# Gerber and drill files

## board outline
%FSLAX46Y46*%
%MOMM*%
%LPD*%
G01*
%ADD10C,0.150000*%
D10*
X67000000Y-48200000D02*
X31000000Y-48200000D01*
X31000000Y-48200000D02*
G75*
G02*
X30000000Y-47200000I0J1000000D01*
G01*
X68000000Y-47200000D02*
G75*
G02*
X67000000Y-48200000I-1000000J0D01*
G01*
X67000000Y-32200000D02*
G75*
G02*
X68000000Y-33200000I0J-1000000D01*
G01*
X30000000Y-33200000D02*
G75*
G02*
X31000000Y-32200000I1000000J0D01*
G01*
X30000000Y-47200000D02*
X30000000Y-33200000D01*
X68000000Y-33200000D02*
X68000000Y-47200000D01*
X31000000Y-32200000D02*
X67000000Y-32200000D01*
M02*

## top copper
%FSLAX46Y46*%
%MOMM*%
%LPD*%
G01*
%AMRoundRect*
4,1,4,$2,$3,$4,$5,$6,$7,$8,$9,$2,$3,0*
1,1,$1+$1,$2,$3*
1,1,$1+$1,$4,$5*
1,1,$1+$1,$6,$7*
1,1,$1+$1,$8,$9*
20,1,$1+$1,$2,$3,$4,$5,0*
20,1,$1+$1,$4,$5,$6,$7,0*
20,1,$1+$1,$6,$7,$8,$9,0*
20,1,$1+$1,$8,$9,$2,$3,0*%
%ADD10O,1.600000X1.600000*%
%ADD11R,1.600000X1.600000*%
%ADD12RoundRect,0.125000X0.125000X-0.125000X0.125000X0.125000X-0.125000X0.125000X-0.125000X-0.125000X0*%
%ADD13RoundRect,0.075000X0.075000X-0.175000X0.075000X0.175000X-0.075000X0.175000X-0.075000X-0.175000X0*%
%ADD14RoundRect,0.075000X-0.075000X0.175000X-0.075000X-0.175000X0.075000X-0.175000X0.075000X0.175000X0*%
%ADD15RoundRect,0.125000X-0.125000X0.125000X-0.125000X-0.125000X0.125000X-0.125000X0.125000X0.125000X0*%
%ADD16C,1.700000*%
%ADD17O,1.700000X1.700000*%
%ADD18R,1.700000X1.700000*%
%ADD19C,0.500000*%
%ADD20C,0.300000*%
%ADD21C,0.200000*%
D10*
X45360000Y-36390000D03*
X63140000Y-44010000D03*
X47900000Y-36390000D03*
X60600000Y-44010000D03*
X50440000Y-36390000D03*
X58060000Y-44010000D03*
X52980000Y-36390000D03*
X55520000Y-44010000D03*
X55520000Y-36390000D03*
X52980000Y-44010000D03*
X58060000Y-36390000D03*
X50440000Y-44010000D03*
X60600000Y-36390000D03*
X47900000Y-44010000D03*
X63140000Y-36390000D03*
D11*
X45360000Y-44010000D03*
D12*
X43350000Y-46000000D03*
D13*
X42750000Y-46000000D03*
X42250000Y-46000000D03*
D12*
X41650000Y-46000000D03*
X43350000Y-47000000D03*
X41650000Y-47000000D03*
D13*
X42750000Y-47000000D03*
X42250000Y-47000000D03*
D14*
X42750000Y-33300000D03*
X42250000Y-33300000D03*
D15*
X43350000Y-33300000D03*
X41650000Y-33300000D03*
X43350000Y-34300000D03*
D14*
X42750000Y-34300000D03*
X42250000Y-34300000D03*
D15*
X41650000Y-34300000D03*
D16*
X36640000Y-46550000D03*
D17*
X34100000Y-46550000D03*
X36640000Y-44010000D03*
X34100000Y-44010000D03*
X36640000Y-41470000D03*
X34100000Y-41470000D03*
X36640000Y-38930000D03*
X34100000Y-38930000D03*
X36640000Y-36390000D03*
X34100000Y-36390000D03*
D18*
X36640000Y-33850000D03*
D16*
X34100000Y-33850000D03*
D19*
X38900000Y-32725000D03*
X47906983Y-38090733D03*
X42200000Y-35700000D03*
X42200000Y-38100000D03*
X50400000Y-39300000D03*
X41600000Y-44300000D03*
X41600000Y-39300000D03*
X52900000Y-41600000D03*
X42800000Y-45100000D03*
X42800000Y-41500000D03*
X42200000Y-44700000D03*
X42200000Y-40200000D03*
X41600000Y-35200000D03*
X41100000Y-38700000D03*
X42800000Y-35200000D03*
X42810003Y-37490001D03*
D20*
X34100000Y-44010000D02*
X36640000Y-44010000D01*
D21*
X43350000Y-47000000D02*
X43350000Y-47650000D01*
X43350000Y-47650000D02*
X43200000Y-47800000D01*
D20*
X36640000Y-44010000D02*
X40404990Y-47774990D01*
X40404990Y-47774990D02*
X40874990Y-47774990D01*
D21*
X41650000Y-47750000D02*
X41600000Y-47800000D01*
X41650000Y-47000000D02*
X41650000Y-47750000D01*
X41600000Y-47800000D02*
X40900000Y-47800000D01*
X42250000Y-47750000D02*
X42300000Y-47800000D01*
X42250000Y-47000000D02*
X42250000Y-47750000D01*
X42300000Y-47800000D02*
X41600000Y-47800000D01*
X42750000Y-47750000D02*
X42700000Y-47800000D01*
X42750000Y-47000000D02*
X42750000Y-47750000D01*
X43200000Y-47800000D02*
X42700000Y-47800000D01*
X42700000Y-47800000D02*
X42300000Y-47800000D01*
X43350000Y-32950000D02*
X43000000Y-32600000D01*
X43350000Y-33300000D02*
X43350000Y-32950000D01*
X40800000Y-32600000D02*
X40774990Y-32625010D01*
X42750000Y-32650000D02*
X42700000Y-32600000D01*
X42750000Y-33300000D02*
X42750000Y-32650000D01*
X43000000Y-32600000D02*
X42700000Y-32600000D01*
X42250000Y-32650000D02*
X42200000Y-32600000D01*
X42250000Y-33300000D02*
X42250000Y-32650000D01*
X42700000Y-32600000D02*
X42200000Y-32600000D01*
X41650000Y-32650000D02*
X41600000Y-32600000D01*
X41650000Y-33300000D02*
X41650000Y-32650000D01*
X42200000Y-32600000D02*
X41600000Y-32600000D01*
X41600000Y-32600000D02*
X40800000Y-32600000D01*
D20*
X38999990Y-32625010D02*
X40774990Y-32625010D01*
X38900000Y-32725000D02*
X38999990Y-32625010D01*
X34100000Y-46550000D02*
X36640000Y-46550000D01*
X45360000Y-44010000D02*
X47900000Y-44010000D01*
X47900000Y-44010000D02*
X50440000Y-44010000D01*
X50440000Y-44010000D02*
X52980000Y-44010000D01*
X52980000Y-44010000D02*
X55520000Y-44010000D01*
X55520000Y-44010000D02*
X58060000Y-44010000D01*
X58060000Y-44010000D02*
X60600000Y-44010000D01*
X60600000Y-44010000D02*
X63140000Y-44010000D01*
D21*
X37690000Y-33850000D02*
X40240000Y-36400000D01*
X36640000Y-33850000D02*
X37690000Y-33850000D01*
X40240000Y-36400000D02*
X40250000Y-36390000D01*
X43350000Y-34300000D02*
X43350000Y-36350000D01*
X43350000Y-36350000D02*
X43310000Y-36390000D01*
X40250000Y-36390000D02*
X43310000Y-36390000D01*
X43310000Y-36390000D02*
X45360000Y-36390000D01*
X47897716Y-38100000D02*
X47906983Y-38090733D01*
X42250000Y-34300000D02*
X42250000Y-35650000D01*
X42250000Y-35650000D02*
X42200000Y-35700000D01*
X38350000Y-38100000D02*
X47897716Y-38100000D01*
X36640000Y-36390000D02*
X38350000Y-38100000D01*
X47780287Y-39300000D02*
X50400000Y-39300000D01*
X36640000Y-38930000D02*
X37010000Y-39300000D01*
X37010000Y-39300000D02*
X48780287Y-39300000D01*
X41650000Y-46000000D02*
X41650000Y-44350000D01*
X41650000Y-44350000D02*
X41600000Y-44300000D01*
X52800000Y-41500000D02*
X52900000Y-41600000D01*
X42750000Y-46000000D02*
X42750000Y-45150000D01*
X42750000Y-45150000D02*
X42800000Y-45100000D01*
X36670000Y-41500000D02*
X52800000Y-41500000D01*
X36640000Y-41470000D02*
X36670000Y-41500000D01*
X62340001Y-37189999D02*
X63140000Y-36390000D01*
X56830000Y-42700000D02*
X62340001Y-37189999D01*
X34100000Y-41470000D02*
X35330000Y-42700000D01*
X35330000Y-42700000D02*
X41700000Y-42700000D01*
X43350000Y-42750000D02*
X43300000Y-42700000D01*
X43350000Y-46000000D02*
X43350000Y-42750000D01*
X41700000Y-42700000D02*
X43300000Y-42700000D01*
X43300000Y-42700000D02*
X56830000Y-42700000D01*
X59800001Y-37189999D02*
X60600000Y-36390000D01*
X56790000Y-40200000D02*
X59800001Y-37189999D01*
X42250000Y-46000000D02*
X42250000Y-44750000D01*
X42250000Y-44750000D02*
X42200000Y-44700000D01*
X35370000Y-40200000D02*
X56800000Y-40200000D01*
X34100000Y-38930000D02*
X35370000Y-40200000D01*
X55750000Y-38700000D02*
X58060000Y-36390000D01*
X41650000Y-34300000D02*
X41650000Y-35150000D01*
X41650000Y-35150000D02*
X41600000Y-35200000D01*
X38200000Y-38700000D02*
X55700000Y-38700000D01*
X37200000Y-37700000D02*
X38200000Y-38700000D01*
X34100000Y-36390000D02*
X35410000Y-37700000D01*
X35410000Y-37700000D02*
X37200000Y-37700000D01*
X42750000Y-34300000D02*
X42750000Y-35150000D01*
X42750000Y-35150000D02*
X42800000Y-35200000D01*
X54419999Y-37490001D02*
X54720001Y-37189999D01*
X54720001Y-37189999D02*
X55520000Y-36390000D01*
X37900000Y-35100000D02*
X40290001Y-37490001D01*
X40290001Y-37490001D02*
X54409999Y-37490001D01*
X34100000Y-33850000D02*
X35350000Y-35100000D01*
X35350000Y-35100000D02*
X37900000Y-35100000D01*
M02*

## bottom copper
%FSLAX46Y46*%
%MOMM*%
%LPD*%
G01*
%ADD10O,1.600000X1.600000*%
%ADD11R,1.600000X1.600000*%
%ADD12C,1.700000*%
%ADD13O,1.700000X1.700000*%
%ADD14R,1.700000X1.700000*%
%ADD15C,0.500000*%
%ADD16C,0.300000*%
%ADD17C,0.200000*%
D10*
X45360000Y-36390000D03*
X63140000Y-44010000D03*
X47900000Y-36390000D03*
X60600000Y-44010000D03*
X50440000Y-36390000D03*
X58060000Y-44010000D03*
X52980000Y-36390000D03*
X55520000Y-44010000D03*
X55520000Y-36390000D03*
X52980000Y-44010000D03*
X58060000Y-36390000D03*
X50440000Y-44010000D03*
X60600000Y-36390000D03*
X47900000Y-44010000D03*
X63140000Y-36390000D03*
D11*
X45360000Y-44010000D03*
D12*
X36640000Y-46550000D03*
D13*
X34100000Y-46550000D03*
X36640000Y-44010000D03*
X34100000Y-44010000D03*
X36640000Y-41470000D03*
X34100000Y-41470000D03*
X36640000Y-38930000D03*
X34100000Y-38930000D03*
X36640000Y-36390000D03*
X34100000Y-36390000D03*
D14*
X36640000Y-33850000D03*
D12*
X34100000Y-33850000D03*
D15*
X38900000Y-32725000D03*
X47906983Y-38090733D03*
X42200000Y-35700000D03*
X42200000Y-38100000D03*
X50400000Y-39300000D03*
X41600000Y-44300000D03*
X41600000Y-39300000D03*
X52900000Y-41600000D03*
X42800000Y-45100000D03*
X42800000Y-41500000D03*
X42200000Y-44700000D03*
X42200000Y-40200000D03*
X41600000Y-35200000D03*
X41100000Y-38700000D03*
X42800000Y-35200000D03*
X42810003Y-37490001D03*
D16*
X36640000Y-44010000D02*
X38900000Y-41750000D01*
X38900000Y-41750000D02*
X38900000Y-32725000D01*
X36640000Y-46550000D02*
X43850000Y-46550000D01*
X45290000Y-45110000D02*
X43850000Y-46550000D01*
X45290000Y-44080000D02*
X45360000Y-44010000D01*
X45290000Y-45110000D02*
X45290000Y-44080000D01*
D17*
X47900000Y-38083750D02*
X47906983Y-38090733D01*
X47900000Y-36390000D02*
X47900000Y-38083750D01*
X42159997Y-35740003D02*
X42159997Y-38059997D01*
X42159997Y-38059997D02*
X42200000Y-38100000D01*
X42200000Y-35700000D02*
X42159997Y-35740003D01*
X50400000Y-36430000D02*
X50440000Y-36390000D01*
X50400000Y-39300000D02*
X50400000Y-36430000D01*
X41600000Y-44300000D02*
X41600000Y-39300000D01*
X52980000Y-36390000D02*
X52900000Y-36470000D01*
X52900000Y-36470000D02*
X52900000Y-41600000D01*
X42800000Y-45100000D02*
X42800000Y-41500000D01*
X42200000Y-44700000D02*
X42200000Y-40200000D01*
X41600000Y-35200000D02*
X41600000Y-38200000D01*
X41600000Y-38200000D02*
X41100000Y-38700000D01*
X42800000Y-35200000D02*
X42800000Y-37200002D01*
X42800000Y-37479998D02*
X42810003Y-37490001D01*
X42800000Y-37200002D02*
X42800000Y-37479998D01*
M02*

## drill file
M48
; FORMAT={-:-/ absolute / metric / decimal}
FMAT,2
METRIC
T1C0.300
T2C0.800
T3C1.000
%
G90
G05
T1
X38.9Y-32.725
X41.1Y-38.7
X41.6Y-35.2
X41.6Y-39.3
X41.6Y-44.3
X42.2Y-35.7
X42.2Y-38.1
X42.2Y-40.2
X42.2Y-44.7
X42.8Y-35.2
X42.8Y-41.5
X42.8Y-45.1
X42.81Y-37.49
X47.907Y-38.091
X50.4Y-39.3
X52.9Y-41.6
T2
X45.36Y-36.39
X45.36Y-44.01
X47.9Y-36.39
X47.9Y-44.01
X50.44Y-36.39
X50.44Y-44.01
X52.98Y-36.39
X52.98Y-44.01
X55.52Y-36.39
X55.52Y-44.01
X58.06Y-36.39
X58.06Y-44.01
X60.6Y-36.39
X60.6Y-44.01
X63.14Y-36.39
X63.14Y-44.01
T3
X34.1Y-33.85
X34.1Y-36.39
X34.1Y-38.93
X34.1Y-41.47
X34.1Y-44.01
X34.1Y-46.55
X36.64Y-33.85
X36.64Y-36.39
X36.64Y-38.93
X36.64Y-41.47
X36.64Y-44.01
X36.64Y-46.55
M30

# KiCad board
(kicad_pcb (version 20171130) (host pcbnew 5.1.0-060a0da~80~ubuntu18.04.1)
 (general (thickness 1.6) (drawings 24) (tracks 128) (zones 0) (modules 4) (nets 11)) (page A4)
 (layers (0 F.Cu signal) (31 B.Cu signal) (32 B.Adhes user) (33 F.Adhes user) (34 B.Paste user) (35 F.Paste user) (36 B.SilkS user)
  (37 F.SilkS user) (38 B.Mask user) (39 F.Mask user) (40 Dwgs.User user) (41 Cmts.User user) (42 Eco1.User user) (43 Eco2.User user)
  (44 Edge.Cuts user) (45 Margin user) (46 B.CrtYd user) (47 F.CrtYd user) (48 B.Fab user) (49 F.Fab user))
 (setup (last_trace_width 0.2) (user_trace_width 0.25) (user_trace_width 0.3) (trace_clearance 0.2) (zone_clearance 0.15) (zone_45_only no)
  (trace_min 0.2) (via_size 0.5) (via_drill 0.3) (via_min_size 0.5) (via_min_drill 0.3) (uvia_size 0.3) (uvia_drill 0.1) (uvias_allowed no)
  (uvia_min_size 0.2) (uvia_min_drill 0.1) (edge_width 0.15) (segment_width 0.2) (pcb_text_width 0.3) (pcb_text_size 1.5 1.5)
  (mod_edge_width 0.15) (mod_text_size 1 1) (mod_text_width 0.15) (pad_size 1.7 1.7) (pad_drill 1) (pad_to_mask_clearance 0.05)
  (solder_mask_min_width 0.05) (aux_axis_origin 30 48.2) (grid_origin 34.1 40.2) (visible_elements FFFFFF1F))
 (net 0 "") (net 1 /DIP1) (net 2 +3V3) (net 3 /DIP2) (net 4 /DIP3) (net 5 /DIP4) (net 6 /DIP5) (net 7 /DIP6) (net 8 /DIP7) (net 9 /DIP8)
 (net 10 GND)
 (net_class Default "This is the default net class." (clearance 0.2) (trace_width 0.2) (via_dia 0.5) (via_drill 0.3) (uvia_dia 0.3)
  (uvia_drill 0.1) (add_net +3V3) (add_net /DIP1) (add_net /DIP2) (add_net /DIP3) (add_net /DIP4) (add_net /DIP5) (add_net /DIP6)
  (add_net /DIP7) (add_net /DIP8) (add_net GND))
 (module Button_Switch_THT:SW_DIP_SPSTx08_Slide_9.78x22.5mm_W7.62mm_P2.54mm (layer F.Cu) (at 45.36 44.01 90)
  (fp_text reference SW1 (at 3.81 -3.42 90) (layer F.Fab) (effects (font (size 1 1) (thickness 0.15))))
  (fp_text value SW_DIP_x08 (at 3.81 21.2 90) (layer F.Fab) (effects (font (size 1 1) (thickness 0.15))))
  (pad 16 thru_hole oval (at 7.62 0 90) (size 1.6 1.6) (drill 0.8) (layers *.Cu *.Mask) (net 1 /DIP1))
  (pad 8 thru_hole oval (at 0 17.78 90) (size 1.6 1.6) (drill 0.8) (layers *.Cu *.Mask) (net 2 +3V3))
  (pad 15 thru_hole oval (at 7.62 2.54 90) (size 1.6 1.6) (drill 0.8) (layers *.Cu *.Mask) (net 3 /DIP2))
  (pad 7 thru_hole oval (at 0 15.24 90) (size 1.6 1.6) (drill 0.8) (layers *.Cu *.Mask) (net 2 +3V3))
  (pad 14 thru_hole oval (at 7.62 5.08 90) (size 1.6 1.6) (drill 0.8) (layers *.Cu *.Mask) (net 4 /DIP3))
  (pad 6 thru_hole oval (at 0 12.7 90) (size 1.6 1.6) (drill 0.8) (layers *.Cu *.Mask) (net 2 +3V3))
  (pad 13 thru_hole oval (at 7.62 7.62 90) (size 1.6 1.6) (drill 0.8) (layers *.Cu *.Mask) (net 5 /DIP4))
  (pad 5 thru_hole oval (at 0 10.16 90) (size 1.6 1.6) (drill 0.8) (layers *.Cu *.Mask) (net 2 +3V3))
  (pad 12 thru_hole oval (at 7.62 10.16 90) (size 1.6 1.6) (drill 0.8) (layers *.Cu *.Mask) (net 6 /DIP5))
  (pad 4 thru_hole oval (at 0 7.62 90) (size 1.6 1.6) (drill 0.8) (layers *.Cu *.Mask) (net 2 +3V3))
  (pad 11 thru_hole oval (at 7.62 12.7 90) (size 1.6 1.6) (drill 0.8) (layers *.Cu *.Mask) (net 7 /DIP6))
  (pad 3 thru_hole oval (at 0 5.08 90) (size 1.6 1.6) (drill 0.8) (layers *.Cu *.Mask) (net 2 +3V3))
  (pad 10 thru_hole oval (at 7.62 15.24 90) (size 1.6 1.6) (drill 0.8) (layers *.Cu *.Mask) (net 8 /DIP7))
  (pad 2 thru_hole oval (at 0 2.54 90) (size 1.6 1.6) (drill 0.8) (layers *.Cu *.Mask) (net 2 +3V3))
  (pad 9 thru_hole oval (at 7.62 17.78 90) (size 1.6 1.6) (drill 0.8) (layers *.Cu *.Mask) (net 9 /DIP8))
  (pad 1 thru_hole rect (at 0 0 90) (size 1.6 1.6) (drill 0.8) (layers *.Cu *.Mask) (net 2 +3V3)))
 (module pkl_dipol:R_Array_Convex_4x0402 (layer F.Cu) (at 42.5 46.5 90) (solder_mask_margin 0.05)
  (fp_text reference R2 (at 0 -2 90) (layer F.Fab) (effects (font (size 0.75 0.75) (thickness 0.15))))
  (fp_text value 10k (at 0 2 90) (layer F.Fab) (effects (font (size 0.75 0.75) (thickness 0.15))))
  (pad 8 smd roundrect (at 0.5 0.85 90) (size 0.5 0.5) (layers F.Cu F.Paste F.Mask) (roundrect_rratio 0.25) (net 9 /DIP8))
  (pad 6 smd roundrect (at 0.5 0.25 90) (size 0.5 0.3) (layers F.Cu F.Paste F.Mask) (roundrect_rratio 0.25) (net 5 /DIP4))
  (pad 4 smd roundrect (at 0.5 -0.25 90) (size 0.5 0.3) (layers F.Cu F.Paste F.Mask) (roundrect_rratio 0.25) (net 8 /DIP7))
  (pad 2 smd roundrect (at 0.5 -0.85 90) (size 0.5 0.5) (layers F.Cu F.Paste F.Mask) (roundrect_rratio 0.25) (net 4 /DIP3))
  (pad 7 smd roundrect (at -0.5 0.85 90) (size 0.5 0.5) (layers F.Cu F.Paste F.Mask) (roundrect_rratio 0.25) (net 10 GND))
  (pad 1 smd roundrect (at -0.5 -0.85 90) (size 0.5 0.5) (layers F.Cu F.Paste F.Mask) (roundrect_rratio 0.25) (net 10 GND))
  (pad 5 smd roundrect (at -0.5 0.25 90) (size 0.5 0.3) (layers F.Cu F.Paste F.Mask) (roundrect_rratio 0.25) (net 10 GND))
  (pad 3 smd roundrect (at -0.5 -0.25 90) (size 0.5 0.3) (layers F.Cu F.Paste F.Mask) (roundrect_rratio 0.25) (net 10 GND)))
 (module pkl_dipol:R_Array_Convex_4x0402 (layer F.Cu) (at 42.5 33.8 270) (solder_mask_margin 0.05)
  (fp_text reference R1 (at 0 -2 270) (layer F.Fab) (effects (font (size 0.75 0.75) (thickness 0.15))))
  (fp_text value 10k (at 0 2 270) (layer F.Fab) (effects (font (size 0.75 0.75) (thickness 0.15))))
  (pad 3 smd roundrect (at -0.5 -0.25 270) (size 0.5 0.3) (layers F.Cu F.Paste F.Mask) (roundrect_rratio 0.25) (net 10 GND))
  (pad 5 smd roundrect (at -0.5 0.25 270) (size 0.5 0.3) (layers F.Cu F.Paste F.Mask) (roundrect_rratio 0.25) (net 10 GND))
  (pad 1 smd roundrect (at -0.5 -0.85 270) (size 0.5 0.5) (layers F.Cu F.Paste F.Mask) (roundrect_rratio 0.25) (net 10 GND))
  (pad 7 smd roundrect (at -0.5 0.85 270) (size 0.5 0.5) (layers F.Cu F.Paste F.Mask) (roundrect_rratio 0.25) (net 10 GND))
  (pad 2 smd roundrect (at 0.5 -0.85 270) (size 0.5 0.5) (layers F.Cu F.Paste F.Mask) (roundrect_rratio 0.25) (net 1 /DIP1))
  (pad 4 smd roundrect (at 0.5 -0.25 270) (size 0.5 0.3) (layers F.Cu F.Paste F.Mask) (roundrect_rratio 0.25) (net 6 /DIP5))
  (pad 6 smd roundrect (at 0.5 0.25 270) (size 0.5 0.3) (layers F.Cu F.Paste F.Mask) (roundrect_rratio 0.25) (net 3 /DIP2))
  (pad 8 smd roundrect (at 0.5 0.85 270) (size 0.5 0.5) (layers F.Cu F.Paste F.Mask) (roundrect_rratio 0.25) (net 7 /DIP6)))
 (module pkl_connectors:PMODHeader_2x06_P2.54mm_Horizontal (layer F.Cu) (at 36.64 46.55 180)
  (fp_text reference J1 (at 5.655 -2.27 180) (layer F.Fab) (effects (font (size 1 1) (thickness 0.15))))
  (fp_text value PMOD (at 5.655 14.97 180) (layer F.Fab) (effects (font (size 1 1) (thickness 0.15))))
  (pad 6 thru_hole circle (at 0 0 180) (size 1.7 1.7) (drill 1) (layers *.Cu *.Mask) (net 2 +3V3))
  (pad 12 thru_hole oval (at 2.54 0 180) (size 1.7 1.7) (drill 1) (layers *.Cu *.Mask) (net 2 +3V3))
  (pad 5 thru_hole oval (at 0 2.54 180) (size 1.7 1.7) (drill 1) (layers *.Cu *.Mask) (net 10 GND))
  (pad 11 thru_hole oval (at 2.54 2.54 180) (size 1.7 1.7) (drill 1) (layers *.Cu *.Mask) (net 10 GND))
  (pad 4 thru_hole oval (at 0 5.08 180) (size 1.7 1.7) (drill 1) (layers *.Cu *.Mask) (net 5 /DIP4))
  (pad 10 thru_hole oval (at 2.54 5.08 180) (size 1.7 1.7) (drill 1) (layers *.Cu *.Mask) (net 9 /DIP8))
  (pad 3 thru_hole oval (at 0 7.62 180) (size 1.7 1.7) (drill 1) (layers *.Cu *.Mask) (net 4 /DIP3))
  (pad 9 thru_hole oval (at 2.54 7.62 180) (size 1.7 1.7) (drill 1) (layers *.Cu *.Mask) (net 8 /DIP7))
  (pad 2 thru_hole oval (at 0 10.16 180) (size 1.7 1.7) (drill 1) (layers *.Cu *.Mask) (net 3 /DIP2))
  (pad 8 thru_hole oval (at 2.54 10.16 180) (size 1.7 1.7) (drill 1) (layers *.Cu *.Mask) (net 7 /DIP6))
  (pad 1 thru_hole rect (at 0 12.7 180) (size 1.7 1.7) (drill 1) (layers *.Cu *.Mask) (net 1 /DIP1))
  (pad 7 thru_hole circle (at 2.54 12.7 180) (size 1.7 1.7) (drill 1) (layers *.Cu *.Mask) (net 6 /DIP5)))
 (gr_line (start 67 48.2) (end 31 48.2) (layer Edge.Cuts) (width 0.15))
 (gr_arc (start 31 47.2) (end 30 47.2) (angle -90) (layer Edge.Cuts) (width 0.15))
 (gr_arc (start 67 47.2) (end 67 48.2) (angle -90) (layer Edge.Cuts) (width 0.15))
 (gr_arc (start 67 33.2) (end 68 33.2) (angle -90) (layer Edge.Cuts) (width 0.15))
 (gr_arc (start 31 33.2) (end 31 32.2) (angle -90) (layer Edge.Cuts) (width 0.15))
 (gr_line (start 30 47.2) (end 30 33.2) (layer Edge.Cuts) (width 0.15))
 (gr_line (start 68 33.2) (end 68 47.2) (layer Edge.Cuts) (width 0.15))
 (gr_line (start 31 32.2) (end 67 32.2) (layer Edge.Cuts) (width 0.15))
 (segment (start 34.1 44.01) (end 36.64 44.01) (width 0.3) (layer F.Cu) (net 10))
 (segment (start 43.35 47) (end 43.35 47.65) (width 0.2) (layer F.Cu) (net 10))
 (segment (start 43.35 47.65) (end 43.2 47.8) (width 0.2) (layer F.Cu) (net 10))
 (segment (start 36.64 44.01) (end 40.40499 47.77499) (width 0.3) (layer F.Cu) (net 10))
 (segment (start 40.40499 47.77499) (end 40.87499 47.77499) (width 0.3) (layer F.Cu) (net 10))
 (segment (start 41.65 47.75) (end 41.6 47.8) (width 0.2) (layer F.Cu) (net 10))
 (segment (start 41.65 47) (end 41.65 47.75) (width 0.2) (layer F.Cu) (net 10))
 (segment (start 41.6 47.8) (end 40.9 47.8) (width 0.2) (layer F.Cu) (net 10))
 (segment (start 42.25 47.75) (end 42.3 47.8) (width 0.2) (layer F.Cu) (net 10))
 (segment (start 42.25 47) (end 42.25 47.75) (width 0.2) (layer F.Cu) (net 10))
 (segment (start 42.3 47.8) (end 41.6 47.8) (width 0.2) (layer F.Cu) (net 10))
 (segment (start 42.75 47.75) (end 42.7 47.8) (width 0.2) (layer F.Cu) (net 10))
 (segment (start 42.75 47) (end 42.75 47.75) (width 0.2) (layer F.Cu) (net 10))
 (segment (start 43.2 47.8) (end 42.7 47.8) (width 0.2) (layer F.Cu) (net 10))
 (segment (start 42.7 47.8) (end 42.3 47.8) (width 0.2) (layer F.Cu) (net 10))
 (via (at 38.9 32.725) (size 0.5) (drill 0.3) (layers F.Cu B.Cu) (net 10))
 (segment (start 36.64 44.01) (end 38.9 41.75) (width 0.3) (layer B.Cu) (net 10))
 (segment (start 38.9 41.75) (end 38.9 32.725) (width 0.3) (layer B.Cu) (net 10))
 (segment (start 43.35 32.95) (end 43 32.6) (width 0.2) (layer F.Cu) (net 10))
 (segment (start 43.35 33.3) (end 43.35 32.95) (width 0.2) (layer F.Cu) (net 10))
 (segment (start 40.8 32.6) (end 40.77499 32.62501) (width 0.2) (layer F.Cu) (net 10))
 (segment (start 42.75 32.65) (end 42.7 32.6) (width 0.2) (layer F.Cu) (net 10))
 (segment (start 42.75 33.3) (end 42.75 32.65) (width 0.2) (layer F.Cu) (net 10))
 (segment (start 43 32.6) (end 42.7 32.6) (width 0.2) (layer F.Cu) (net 10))
 (segment (start 42.25 32.65) (end 42.2 32.6) (width 0.2) (layer F.Cu) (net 10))
 (segment (start 42.25 33.3) (end 42.25 32.65) (width 0.2) (layer F.Cu) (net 10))
 (segment (start 42.7 32.6) (end 42.2 32.6) (width 0.2) (layer F.Cu) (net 10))
 (segment (start 41.65 32.65) (end 41.6 32.6) (width 0.2) (layer F.Cu) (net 10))
 (segment (start 41.65 33.3) (end 41.65 32.65) (width 0.2) (layer F.Cu) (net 10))
 (segment (start 42.2 32.6) (end 41.6 32.6) (width 0.2) (layer F.Cu) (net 10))
 (segment (start 41.6 32.6) (end 40.8 32.6) (width 0.2) (layer F.Cu) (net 10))
 (segment (start 38.99999 32.62501) (end 40.77499 32.62501) (width 0.3) (layer F.Cu) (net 10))
 (segment (start 38.9 32.725) (end 38.99999 32.62501) (width 0.3) (layer F.Cu) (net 10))
 (segment (start 34.1 46.55) (end 36.64 46.55) (width 0.3) (layer F.Cu) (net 2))
 (segment (start 45.36 44.01) (end 47.9 44.01) (width 0.3) (layer F.Cu) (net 2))
 (segment (start 47.9 44.01) (end 50.44 44.01) (width 0.3) (layer F.Cu) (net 2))
 (segment (start 50.44 44.01) (end 52.98 44.01) (width 0.3) (layer F.Cu) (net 2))
 (segment (start 52.98 44.01) (end 55.52 44.01) (width 0.3) (layer F.Cu) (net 2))
 (segment (start 55.52 44.01) (end 58.06 44.01) (width 0.3) (layer F.Cu) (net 2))
 (segment (start 58.06 44.01) (end 60.6 44.01) (width 0.3) (layer F.Cu) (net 2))
 (segment (start 60.6 44.01) (end 63.14 44.01) (width 0.3) (layer F.Cu) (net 2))
 (segment (start 36.64 46.55) (end 43.85 46.55) (width 0.3) (layer B.Cu) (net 2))
 (segment (start 45.29 45.11) (end 43.85 46.55) (width 0.3) (layer B.Cu) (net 2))
 (segment (start 45.29 44.08) (end 45.36 44.01) (width 0.3) (layer B.Cu) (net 2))
 (segment (start 45.29 45.11) (end 45.29 44.08) (width 0.3) (layer B.Cu) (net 2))
 (segment (start 37.69 33.85) (end 40.24 36.4) (width 0.2) (layer F.Cu) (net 1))
 (segment (start 36.64 33.85) (end 37.69 33.85) (width 0.2) (layer F.Cu) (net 1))
 (segment (start 40.24 36.4) (end 40.25 36.39) (width 0.2) (layer F.Cu) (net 1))
 (segment (start 43.35 34.3) (end 43.35 36.35) (width 0.2) (layer F.Cu) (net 1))
 (segment (start 43.35 36.35) (end 43.31 36.39) (width 0.2) (layer F.Cu) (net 1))
 (segment (start 40.25 36.39) (end 43.31 36.39) (width 0.2) (layer F.Cu) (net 1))
 (segment (start 43.31 36.39) (end 45.36 36.39) (width 0.2) (layer F.Cu) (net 1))
 (via (at 47.906983 38.090733) (size 0.5) (drill 0.3) (layers F.Cu B.Cu) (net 3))
 (segment (start 47.9 38.08375) (end 47.906983 38.090733) (width 0.2) (layer B.Cu) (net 3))
 (segment (start 47.9 36.39) (end 47.9 38.08375) (width 0.2) (layer B.Cu) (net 3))
 (segment (start 47.897716 38.1) (end 47.906983 38.090733) (width 0.2) (layer F.Cu) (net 3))
 (via (at 42.2 35.7) (size 0.5) (drill 0.3) (layers F.Cu B.Cu) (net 3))
 (segment (start 42.25 34.3) (end 42.25 35.65) (width 0.2) (layer F.Cu) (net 3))
 (segment (start 42.25 35.65) (end 42.2 35.7) (width 0.2) (layer F.Cu) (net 3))
 (via (at 42.2 38.1) (size 0.5) (drill 0.3) (layers F.Cu B.Cu) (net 3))
 (segment (start 42.159997 35.740003) (end 42.159997 38.059997) (width 0.2) (layer B.Cu) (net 3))
 (segment (start 42.159997 38.059997) (end 42.2 38.1) (width 0.2) (layer B.Cu) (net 3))
 (segment (start 42.2 35.7) (end 42.159997 35.740003) (width 0.2) (layer B.Cu) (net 3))
 (segment (start 38.35 38.1) (end 47.897716 38.1) (width 0.2) (layer F.Cu) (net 3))
 (segment (start 36.64 36.39) (end 38.35 38.1) (width 0.2) (layer F.Cu) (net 3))
 (via (at 50.4 39.3) (size 0.5) (drill 0.3) (layers F.Cu B.Cu) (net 4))
 (segment (start 50.4 36.43) (end 50.44 36.39) (width 0.2) (layer B.Cu) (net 4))
 (segment (start 50.4 39.3) (end 50.4 36.43) (width 0.2) (layer B.Cu) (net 4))
 (segment (start 47.780287 39.3) (end 50.4 39.3) (width 0.2) (layer F.Cu) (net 4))
 (segment (start 36.64 38.93) (end 37.01 39.3) (width 0.2) (layer F.Cu) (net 4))
 (segment (start 37.01 39.3) (end 48.780287 39.3) (width 0.2) (layer F.Cu) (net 4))
 (via (at 41.6 44.3) (size 0.5) (drill 0.3) (layers F.Cu B.Cu) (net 4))
 (segment (start 41.65 46) (end 41.65 44.35) (width 0.2) (layer F.Cu) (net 4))
 (segment (start 41.65 44.35) (end 41.6 44.3) (width 0.2) (layer F.Cu) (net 4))
 (via (at 41.6 39.3) (size 0.5) (drill 0.3) (layers F.Cu B.Cu) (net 4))
 (segment (start 41.6 44.3) (end 41.6 39.3) (width 0.2) (layer B.Cu) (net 4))
 (segment (start 52.8 41.5) (end 52.9 41.6) (width 0.2) (layer F.Cu) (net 5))
 (via (at 52.9 41.6) (size 0.5) (drill 0.3) (layers F.Cu B.Cu) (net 5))
 (segment (start 52.98 36.39) (end 52.9 36.47) (width 0.2) (layer B.Cu) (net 5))
 (segment (start 52.9 36.47) (end 52.9 41.6) (width 0.2) (layer B.Cu) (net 5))
 (via (at 42.8 45.1) (size 0.5) (drill 0.3) (layers F.Cu B.Cu) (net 5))
 (segment (start 42.75 46) (end 42.75 45.15) (width 0.2) (layer F.Cu) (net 5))
 (segment (start 42.75 45.15) (end 42.8 45.1) (width 0.2) (layer F.Cu) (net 5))
 (via (at 42.8 41.5) (size 0.5) (drill 0.3) (layers F.Cu B.Cu) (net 5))
 (segment (start 42.8 45.1) (end 42.8 41.5) (width 0.2) (layer B.Cu) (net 5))
 (segment (start 36.67 41.5) (end 52.8 41.5) (width 0.2) (layer F.Cu) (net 5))
 (segment (start 36.64 41.47) (end 36.67 41.5) (width 0.2) (layer F.Cu) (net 5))
 (segment (start 62.340001 37.189999) (end 63.14 36.39) (width 0.2) (layer F.Cu) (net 9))
 (segment (start 56.83 42.7) (end 62.340001 37.189999) (width 0.2) (layer F.Cu) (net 9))
 (segment (start 34.1 41.47) (end 35.33 42.7) (width 0.2) (layer F.Cu) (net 9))
 (segment (start 35.33 42.7) (end 41.7 42.7) (width 0.2) (layer F.Cu) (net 9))
 (segment (start 43.35 42.75) (end 43.3 42.7) (width 0.2) (layer F.Cu) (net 9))
 (segment (start 43.35 46) (end 43.35 42.75) (width 0.2) (layer F.Cu) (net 9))
 (segment (start 41.7 42.7) (end 43.3 42.7) (width 0.2) (layer F.Cu) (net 9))
 (segment (start 43.3 42.7) (end 56.83 42.7) (width 0.2) (layer F.Cu) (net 9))
 (segment (start 59.800001 37.189999) (end 60.6 36.39) (width 0.2) (layer F.Cu) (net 8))
 (segment (start 56.79 40.2) (end 59.800001 37.189999) (width 0.2) (layer F.Cu) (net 8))
 (via (at 42.2 44.7) (size 0.5) (drill 0.3) (layers F.Cu B.Cu) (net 8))
 (segment (start 42.25 46) (end 42.25 44.75) (width 0.2) (layer F.Cu) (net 8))
 (segment (start 42.25 44.75) (end 42.2 44.7) (width 0.2) (layer F.Cu) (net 8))
 (via (at 42.2 40.2) (size 0.5) (drill 0.3) (layers F.Cu B.Cu) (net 8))
 (segment (start 42.2 44.7) (end 42.2 40.2) (width 0.2) (layer B.Cu) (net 8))
 (segment (start 35.37 40.2) (end 56.8 40.2) (width 0.2) (layer F.Cu) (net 8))
 (segment (start 34.1 38.93) (end 35.37 40.2) (width 0.2) (layer F.Cu) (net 8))
 (segment (start 55.75 38.7) (end 58.06 36.39) (width 0.2) (layer F.Cu) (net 7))
 (via (at 41.6 35.2) (size 0.5) (drill 0.3) (layers F.Cu B.Cu) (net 7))
 (segment (start 41.65 34.3) (end 41.65 35.15) (width 0.2) (layer F.Cu) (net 7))
 (segment (start 41.65 35.15) (end 41.6 35.2) (width 0.2) (layer F.Cu) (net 7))
 (segment (start 41.6 35.2) (end 41.6 38.2) (width 0.2) (layer B.Cu) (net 7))
 (via (at 41.1 38.7) (size 0.5) (drill 0.3) (layers F.Cu B.Cu) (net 7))
 (segment (start 41.6 38.2) (end 41.1 38.7) (width 0.2) (layer B.Cu) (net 7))
 (segment (start 38.2 38.7) (end 55.7 38.7) (width 0.2) (layer F.Cu) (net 7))
 (segment (start 37.2 37.7) (end 38.2 38.7) (width 0.2) (layer F.Cu) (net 7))
 (segment (start 34.1 36.39) (end 35.41 37.7) (width 0.2) (layer F.Cu) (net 7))
 (segment (start 35.41 37.7) (end 37.2 37.7) (width 0.2) (layer F.Cu) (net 7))
 (via (at 42.8 35.2) (size 0.5) (drill 0.3) (layers F.Cu B.Cu) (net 6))
 (segment (start 42.75 34.3) (end 42.75 35.15) (width 0.2) (layer F.Cu) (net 6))
 (segment (start 42.75 35.15) (end 42.8 35.2) (width 0.2) (layer F.Cu) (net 6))
 (segment (start 42.8 35.2) (end 42.8 37.200002) (width 0.2) (layer B.Cu) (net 6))
 (via (at 42.810003 37.490001) (size 0.5) (drill 0.3) (layers F.Cu B.Cu) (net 6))
 (segment (start 42.8 37.479998) (end 42.810003 37.490001) (width 0.2) (layer B.Cu) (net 6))
 (segment (start 42.8 37.200002) (end 42.8 37.479998) (width 0.2) (layer B.Cu) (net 6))
 (segment (start 54.419999 37.490001) (end 54.720001 37.189999) (width 0.2) (layer F.Cu) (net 6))
 (segment (start 54.720001 37.189999) (end 55.52 36.39) (width 0.2) (layer F.Cu) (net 6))
 (segment (start 37.9 35.1) (end 40.290001 37.490001) (width 0.2) (layer F.Cu) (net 6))
 (segment (start 40.290001 37.490001) (end 54.409999 37.490001) (width 0.2) (layer F.Cu) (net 6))
 (segment (start 34.1 33.85) (end 35.35 35.1) (width 0.2) (layer F.Cu) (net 6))
 (segment (start 35.35 35.1) (end 37.9 35.1) (width 0.2) (layer F.Cu) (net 6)))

